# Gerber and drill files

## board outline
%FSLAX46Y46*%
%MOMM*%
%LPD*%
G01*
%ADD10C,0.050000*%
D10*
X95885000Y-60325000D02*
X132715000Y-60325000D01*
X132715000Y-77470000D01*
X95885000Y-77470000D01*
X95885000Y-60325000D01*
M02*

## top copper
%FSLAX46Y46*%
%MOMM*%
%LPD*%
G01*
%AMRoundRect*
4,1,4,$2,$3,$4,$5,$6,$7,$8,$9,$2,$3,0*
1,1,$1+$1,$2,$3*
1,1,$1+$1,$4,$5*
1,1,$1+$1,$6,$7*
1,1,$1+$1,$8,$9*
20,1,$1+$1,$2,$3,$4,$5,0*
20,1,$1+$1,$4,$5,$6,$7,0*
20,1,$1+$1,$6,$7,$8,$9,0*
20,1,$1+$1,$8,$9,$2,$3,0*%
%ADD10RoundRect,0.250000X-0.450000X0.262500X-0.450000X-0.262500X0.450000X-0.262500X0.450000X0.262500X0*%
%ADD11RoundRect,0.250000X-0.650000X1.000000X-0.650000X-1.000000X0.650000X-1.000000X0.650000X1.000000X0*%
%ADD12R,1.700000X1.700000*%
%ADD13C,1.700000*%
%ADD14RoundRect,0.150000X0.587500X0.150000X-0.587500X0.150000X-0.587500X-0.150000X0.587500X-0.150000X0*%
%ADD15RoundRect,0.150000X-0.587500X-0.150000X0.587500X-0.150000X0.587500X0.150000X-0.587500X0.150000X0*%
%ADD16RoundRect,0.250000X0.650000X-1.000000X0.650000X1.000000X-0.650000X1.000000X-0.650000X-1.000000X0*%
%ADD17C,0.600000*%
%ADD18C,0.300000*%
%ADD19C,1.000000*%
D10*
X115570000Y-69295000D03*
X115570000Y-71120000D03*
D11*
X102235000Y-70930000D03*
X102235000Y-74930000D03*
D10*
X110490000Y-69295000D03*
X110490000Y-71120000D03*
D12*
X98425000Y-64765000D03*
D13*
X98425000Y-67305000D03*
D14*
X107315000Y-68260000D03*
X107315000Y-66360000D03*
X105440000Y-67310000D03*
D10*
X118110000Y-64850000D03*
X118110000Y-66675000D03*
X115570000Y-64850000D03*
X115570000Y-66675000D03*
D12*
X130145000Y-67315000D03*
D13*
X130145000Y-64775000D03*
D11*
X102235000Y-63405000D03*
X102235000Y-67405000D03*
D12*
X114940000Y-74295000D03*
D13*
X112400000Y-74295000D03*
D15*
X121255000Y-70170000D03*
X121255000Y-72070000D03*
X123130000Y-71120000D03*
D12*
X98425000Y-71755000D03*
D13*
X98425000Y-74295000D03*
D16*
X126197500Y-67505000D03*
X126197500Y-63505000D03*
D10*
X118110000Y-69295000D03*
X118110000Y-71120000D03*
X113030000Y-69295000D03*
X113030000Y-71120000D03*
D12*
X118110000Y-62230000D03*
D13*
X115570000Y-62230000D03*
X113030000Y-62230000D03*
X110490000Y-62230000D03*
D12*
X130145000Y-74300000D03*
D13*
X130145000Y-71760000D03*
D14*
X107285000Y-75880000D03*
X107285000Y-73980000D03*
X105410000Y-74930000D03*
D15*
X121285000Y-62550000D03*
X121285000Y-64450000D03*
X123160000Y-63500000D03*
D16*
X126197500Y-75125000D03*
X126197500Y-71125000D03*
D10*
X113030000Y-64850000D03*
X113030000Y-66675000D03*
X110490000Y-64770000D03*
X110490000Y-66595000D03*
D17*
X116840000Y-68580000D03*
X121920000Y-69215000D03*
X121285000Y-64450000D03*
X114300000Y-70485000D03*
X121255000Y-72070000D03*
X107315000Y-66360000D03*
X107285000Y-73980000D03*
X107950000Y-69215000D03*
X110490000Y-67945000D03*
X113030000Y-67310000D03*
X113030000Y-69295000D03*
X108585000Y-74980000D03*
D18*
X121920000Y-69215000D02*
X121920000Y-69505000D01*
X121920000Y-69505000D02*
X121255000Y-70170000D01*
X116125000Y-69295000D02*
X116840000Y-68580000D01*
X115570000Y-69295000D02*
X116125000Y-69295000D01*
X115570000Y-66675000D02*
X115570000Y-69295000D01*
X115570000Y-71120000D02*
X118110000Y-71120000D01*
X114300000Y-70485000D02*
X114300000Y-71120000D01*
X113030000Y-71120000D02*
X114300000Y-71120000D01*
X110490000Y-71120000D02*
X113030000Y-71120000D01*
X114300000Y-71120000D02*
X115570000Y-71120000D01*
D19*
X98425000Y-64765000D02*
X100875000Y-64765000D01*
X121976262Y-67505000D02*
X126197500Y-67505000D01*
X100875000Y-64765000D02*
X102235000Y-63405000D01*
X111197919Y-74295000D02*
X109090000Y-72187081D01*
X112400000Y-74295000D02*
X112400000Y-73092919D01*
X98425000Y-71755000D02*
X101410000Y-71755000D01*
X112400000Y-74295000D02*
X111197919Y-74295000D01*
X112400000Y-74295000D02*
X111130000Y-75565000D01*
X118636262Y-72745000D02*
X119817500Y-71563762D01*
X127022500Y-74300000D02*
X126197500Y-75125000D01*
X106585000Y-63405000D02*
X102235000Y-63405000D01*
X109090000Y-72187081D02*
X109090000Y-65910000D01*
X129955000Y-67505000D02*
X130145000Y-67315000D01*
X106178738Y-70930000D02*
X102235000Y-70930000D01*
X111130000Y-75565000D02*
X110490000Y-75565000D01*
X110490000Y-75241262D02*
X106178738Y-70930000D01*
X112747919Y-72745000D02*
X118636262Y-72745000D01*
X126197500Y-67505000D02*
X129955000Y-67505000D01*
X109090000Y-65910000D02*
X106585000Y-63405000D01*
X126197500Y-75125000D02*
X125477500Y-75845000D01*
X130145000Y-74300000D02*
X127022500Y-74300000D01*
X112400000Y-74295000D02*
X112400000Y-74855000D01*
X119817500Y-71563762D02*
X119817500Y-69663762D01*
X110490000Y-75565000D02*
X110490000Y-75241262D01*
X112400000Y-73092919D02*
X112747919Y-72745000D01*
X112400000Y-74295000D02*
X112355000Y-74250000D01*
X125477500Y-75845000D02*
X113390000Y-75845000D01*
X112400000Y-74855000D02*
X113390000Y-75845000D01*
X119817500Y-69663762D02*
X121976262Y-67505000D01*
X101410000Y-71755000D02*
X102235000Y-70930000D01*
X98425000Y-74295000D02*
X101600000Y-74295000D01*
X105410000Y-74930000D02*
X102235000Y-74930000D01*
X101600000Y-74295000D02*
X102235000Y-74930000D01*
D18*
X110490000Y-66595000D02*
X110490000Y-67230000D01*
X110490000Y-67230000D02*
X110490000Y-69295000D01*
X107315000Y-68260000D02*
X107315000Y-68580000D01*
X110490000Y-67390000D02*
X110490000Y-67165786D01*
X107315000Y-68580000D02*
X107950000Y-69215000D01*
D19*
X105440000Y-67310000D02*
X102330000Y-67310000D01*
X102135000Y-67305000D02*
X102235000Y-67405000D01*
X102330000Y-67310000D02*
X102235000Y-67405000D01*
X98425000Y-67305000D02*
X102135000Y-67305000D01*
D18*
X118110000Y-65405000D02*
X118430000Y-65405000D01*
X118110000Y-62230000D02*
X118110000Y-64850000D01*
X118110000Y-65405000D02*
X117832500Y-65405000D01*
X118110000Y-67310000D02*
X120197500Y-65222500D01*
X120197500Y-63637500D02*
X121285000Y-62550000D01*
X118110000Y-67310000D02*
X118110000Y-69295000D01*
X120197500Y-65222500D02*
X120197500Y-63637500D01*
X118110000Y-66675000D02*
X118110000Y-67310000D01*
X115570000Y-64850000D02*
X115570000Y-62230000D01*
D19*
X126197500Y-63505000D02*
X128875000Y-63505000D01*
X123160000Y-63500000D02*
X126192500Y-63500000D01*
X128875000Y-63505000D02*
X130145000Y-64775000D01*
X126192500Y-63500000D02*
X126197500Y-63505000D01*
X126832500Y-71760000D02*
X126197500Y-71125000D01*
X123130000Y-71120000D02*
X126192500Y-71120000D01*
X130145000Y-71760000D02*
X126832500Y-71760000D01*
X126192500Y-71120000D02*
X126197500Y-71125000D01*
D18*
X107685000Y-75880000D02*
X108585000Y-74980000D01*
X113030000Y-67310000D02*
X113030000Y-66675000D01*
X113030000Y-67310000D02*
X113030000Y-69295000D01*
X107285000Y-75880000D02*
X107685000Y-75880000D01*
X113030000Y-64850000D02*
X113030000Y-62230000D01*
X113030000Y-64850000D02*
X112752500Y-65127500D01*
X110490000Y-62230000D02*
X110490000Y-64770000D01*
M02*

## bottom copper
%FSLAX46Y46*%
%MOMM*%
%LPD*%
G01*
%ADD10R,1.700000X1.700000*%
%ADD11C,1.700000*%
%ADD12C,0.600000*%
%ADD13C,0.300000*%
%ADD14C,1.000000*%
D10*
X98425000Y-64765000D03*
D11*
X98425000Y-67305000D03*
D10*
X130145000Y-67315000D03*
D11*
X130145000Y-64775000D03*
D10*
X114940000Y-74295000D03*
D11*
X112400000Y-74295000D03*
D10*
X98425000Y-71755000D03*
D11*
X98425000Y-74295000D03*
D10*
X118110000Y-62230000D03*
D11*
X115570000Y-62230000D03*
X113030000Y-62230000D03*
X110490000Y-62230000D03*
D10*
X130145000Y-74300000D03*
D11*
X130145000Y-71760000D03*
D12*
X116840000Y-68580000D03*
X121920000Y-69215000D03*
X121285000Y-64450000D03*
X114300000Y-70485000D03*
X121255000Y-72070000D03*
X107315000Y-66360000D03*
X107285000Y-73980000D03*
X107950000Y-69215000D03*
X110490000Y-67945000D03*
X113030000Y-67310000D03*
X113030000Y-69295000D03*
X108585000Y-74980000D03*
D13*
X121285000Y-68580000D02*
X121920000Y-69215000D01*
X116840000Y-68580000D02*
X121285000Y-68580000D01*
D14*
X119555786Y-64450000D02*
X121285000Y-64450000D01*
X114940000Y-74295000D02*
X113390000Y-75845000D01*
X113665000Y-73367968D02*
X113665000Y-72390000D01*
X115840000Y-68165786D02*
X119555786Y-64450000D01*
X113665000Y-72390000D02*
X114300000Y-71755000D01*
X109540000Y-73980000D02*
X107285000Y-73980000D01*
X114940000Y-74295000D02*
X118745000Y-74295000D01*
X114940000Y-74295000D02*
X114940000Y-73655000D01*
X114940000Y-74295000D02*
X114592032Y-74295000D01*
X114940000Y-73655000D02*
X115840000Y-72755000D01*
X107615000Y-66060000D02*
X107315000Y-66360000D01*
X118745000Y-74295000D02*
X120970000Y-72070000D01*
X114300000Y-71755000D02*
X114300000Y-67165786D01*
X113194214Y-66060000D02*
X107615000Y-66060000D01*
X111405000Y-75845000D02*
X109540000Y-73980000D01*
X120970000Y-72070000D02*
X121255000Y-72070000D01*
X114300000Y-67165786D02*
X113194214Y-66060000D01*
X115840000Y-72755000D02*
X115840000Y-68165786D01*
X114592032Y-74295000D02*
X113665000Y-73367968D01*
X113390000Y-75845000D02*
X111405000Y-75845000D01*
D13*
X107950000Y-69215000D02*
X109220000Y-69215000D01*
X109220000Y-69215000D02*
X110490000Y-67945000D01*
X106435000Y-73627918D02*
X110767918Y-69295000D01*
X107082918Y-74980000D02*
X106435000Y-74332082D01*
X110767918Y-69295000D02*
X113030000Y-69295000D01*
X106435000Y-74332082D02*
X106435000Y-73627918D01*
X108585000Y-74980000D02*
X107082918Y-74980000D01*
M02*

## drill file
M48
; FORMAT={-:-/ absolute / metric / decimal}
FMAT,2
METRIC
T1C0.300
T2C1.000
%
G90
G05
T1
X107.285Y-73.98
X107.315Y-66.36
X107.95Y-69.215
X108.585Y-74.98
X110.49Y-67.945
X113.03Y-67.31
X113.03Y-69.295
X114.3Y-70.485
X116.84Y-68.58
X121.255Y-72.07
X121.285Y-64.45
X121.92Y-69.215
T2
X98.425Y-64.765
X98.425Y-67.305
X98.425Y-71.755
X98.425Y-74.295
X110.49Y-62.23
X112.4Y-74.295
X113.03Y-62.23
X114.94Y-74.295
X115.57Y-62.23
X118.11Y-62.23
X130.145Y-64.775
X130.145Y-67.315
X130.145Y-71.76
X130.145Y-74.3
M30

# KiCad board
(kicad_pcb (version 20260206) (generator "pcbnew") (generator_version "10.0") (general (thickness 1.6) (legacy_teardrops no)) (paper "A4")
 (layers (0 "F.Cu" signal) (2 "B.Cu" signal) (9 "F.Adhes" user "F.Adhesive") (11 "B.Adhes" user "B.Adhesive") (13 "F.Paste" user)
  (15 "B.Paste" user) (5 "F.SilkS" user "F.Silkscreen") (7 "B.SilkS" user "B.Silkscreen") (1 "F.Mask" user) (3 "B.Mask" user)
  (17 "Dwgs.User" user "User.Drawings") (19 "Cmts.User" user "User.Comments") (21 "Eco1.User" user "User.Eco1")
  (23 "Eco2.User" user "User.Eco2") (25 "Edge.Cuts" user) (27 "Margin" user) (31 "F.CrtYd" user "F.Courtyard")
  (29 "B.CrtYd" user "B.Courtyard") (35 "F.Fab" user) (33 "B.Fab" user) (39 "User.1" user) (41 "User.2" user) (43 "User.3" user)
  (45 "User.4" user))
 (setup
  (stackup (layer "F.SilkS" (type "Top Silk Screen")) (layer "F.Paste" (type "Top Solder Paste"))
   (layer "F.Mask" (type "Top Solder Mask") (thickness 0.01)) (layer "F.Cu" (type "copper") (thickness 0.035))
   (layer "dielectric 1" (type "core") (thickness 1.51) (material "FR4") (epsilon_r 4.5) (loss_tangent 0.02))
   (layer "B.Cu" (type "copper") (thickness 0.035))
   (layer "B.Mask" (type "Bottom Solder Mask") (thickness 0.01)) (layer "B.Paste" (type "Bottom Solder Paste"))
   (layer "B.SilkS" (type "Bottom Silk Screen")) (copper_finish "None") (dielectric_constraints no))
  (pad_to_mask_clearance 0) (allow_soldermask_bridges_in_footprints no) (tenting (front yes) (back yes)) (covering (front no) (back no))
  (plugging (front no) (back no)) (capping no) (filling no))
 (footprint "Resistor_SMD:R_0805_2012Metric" (layer "F.Cu") (at 115.57 70.2075 -90)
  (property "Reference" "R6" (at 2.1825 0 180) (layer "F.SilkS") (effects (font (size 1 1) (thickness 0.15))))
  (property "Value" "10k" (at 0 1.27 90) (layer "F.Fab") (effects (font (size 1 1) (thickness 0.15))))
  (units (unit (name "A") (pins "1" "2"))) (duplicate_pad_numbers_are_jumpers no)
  (pad "1" smd roundrect (at -0.9125 0 270) (size 1.025 1.4) (layers "F.Cu" "F.Mask" "F.Paste") (roundrect_rratio 0.243902)
   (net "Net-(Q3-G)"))
  (pad "2" smd roundrect (at 0.9125 0 270) (size 1.025 1.4) (layers "F.Cu" "F.Mask" "F.Paste") (roundrect_rratio 0.243902) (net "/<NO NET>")))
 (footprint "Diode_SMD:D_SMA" (layer "F.Cu") (at 102.235 72.93 -90)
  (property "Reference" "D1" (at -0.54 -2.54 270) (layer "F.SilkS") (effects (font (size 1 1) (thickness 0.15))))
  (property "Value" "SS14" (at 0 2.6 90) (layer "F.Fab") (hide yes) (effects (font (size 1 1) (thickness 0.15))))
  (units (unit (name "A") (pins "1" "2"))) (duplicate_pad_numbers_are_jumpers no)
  (pad "1" smd roundrect (at -2 0 270) (size 2.5 1.8) (layers "F.Cu" "F.Mask" "F.Paste") (roundrect_rratio 0.1388888889) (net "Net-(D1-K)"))
  (pad "2" smd roundrect (at 2 0 270) (size 2.5 1.8) (layers "F.Cu" "F.Mask" "F.Paste") (roundrect_rratio 0.1388888889) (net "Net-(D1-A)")))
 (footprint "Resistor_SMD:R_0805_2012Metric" (layer "F.Cu") (at 110.49 70.2075 -90)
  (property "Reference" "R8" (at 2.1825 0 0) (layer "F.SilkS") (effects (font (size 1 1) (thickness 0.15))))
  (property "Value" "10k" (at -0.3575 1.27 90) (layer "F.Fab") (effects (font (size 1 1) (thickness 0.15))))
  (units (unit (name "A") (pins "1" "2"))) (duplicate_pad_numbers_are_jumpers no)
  (pad "1" smd roundrect (at -0.9125 0 270) (size 1.025 1.4) (layers "F.Cu" "F.Mask" "F.Paste") (roundrect_rratio 0.243902)
   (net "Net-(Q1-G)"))
  (pad "2" smd roundrect (at 0.9125 0 270) (size 1.025 1.4) (layers "F.Cu" "F.Mask" "F.Paste") (roundrect_rratio 0.243902) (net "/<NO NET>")))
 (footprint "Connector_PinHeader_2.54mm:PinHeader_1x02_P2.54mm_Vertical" (layer "F.Cu") (at 98.425 64.765)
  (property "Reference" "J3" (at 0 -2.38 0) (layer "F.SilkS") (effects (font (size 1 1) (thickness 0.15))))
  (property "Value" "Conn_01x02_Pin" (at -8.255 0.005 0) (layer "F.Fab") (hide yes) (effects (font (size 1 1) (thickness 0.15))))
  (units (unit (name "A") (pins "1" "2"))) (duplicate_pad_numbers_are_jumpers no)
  (pad "1" thru_hole rect (at 0 0) (size 1.7 1.7) (drill 1) (layers "*.Cu" "*.Mask") (remove_unused_layers no) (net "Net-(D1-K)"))
  (pad "2" thru_hole circle (at 0 2.54) (size 1.7 1.7) (drill 1) (layers "*.Cu" "*.Mask") (remove_unused_layers no) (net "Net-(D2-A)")))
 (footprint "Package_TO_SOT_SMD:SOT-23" (layer "F.Cu") (at 106.3775 67.31 180)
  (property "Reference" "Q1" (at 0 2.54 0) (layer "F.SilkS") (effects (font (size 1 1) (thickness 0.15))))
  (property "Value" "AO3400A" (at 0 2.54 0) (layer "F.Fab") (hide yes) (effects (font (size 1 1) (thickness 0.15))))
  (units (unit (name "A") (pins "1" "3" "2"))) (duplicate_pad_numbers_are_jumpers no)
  (pad "1" smd roundrect (at -0.9375 -0.95 180) (size 1.475 0.6) (layers "F.Cu" "F.Mask" "F.Paste") (roundrect_rratio 0.25)
   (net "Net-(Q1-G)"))
  (pad "2" smd roundrect (at -0.9375 0.95 180) (size 1.475 0.6) (layers "F.Cu" "F.Mask" "F.Paste") (roundrect_rratio 0.25) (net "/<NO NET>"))
  (pad "3" smd roundrect (at 0.9375 0 180) (size 1.475 0.6) (layers "F.Cu" "F.Mask" "F.Paste") (roundrect_rratio 0.25) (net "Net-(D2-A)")))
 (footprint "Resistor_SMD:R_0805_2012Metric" (layer "F.Cu") (at 118.11 65.7625 -90)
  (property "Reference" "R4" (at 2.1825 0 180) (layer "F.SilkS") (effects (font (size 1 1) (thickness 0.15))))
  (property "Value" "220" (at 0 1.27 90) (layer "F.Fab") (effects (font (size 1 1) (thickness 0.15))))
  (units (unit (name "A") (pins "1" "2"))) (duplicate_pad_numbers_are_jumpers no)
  (pad "1" smd roundrect (at -0.9125 0 270) (size 1.025 1.4) (layers "F.Cu" "F.Mask" "F.Paste") (roundrect_rratio 0.243902)
   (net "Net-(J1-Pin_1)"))
  (pad "2" smd roundrect (at 0.9125 0 270) (size 1.025 1.4) (layers "F.Cu" "F.Mask" "F.Paste") (roundrect_rratio 0.243902)
   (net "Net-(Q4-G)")))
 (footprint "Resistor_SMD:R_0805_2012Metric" (layer "F.Cu") (at 115.57 65.7625 -90)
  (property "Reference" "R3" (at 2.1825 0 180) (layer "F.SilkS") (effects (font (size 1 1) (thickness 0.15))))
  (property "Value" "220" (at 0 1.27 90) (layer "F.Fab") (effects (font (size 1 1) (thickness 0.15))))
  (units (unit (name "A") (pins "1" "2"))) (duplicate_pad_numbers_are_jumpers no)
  (pad "1" smd roundrect (at -0.9125 0 270) (size 1.025 1.4) (layers "F.Cu" "F.Mask" "F.Paste") (roundrect_rratio 0.243902)
   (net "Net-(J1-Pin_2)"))
  (pad "2" smd roundrect (at 0.9125 0 270) (size 1.025 1.4) (layers "F.Cu" "F.Mask" "F.Paste") (roundrect_rratio 0.243902)
   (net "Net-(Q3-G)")))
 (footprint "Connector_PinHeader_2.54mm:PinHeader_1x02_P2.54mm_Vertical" (layer "F.Cu") (at 130.145 67.315 180)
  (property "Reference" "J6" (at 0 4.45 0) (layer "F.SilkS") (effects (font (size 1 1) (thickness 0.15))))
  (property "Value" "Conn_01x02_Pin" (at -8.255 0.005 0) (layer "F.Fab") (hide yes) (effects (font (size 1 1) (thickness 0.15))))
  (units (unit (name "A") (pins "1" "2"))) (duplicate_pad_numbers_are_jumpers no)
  (pad "1" thru_hole rect (at 0 0 180) (size 1.7 1.7) (drill 1) (layers "*.Cu" "*.Mask") (remove_unused_layers no) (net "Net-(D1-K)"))
  (pad "2" thru_hole circle (at 0 2.54 180) (size 1.7 1.7) (drill 1) (layers "*.Cu" "*.Mask") (remove_unused_layers no) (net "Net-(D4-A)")))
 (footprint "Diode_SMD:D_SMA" (layer "F.Cu") (at 102.235 65.405 -90)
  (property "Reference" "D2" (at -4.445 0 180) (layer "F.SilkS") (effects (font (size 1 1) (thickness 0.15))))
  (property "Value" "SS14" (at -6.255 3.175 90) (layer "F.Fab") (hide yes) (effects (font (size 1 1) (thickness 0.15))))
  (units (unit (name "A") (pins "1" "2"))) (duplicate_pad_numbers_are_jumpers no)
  (pad "1" smd roundrect (at -2 0 270) (size 2.5 1.8) (layers "F.Cu" "F.Mask" "F.Paste") (roundrect_rratio 0.1388888889) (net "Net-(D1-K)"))
  (pad "2" smd roundrect (at 2 0 270) (size 2.5 1.8) (layers "F.Cu" "F.Mask" "F.Paste") (roundrect_rratio 0.1388888889) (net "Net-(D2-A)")))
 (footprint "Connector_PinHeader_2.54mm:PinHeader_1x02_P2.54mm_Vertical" (layer "F.Cu") (at 114.94 74.295 -90)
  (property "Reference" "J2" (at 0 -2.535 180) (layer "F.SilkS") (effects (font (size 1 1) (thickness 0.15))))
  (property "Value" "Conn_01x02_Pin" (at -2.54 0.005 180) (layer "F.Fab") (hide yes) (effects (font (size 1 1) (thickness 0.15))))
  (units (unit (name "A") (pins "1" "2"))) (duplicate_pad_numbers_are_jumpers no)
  (pad "1" thru_hole rect (at 0 0 270) (size 1.7 1.7) (drill 1) (layers "*.Cu" "*.Mask") (remove_unused_layers no) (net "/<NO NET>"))
  (pad "2" thru_hole circle (at 0 2.54 270) (size 1.7 1.7) (drill 1) (layers "*.Cu" "*.Mask") (remove_unused_layers no) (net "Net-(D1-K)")))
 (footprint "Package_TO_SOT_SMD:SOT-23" (layer "F.Cu") (at 122.1925 71.12)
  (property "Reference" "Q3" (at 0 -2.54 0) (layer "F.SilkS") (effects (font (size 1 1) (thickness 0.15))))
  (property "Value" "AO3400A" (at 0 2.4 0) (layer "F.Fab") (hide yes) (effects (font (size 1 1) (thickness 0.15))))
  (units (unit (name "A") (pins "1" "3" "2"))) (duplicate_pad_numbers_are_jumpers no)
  (pad "1" smd roundrect (at -0.9375 -0.95) (size 1.475 0.6) (layers "F.Cu" "F.Mask" "F.Paste") (roundrect_rratio 0.25) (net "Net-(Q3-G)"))
  (pad "2" smd roundrect (at -0.9375 0.95) (size 1.475 0.6) (layers "F.Cu" "F.Mask" "F.Paste") (roundrect_rratio 0.25) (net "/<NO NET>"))
  (pad "3" smd roundrect (at 0.9375 0) (size 1.475 0.6) (layers "F.Cu" "F.Mask" "F.Paste") (roundrect_rratio 0.25) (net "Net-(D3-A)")))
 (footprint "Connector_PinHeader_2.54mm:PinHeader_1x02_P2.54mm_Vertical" (layer "F.Cu") (at 98.425 71.755)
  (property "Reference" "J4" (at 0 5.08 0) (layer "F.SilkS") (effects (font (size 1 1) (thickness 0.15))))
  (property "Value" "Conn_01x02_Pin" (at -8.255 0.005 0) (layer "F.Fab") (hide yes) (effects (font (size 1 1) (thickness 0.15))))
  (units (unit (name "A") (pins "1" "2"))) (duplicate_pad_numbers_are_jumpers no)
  (pad "1" thru_hole rect (at 0 0) (size 1.7 1.7) (drill 1) (layers "*.Cu" "*.Mask") (remove_unused_layers no) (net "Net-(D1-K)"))
  (pad "2" thru_hole circle (at 0 2.54) (size 1.7 1.7) (drill 1) (layers "*.Cu" "*.Mask") (remove_unused_layers no) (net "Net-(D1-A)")))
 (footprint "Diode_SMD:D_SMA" (layer "F.Cu") (at 126.1975 65.505 90)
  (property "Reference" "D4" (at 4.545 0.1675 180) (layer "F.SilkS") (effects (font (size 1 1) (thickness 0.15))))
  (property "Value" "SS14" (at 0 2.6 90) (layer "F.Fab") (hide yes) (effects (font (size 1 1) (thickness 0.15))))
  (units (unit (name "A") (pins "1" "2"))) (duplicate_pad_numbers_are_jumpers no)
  (pad "1" smd roundrect (at -2 0 90) (size 2.5 1.8) (layers "F.Cu" "F.Mask" "F.Paste") (roundrect_rratio 0.1388888889) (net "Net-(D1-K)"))
  (pad "2" smd roundrect (at 2 0 90) (size 2.5 1.8) (layers "F.Cu" "F.Mask" "F.Paste") (roundrect_rratio 0.1388888889) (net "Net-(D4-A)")))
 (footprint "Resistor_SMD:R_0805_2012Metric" (layer "F.Cu") (at 118.11 70.2075 -90)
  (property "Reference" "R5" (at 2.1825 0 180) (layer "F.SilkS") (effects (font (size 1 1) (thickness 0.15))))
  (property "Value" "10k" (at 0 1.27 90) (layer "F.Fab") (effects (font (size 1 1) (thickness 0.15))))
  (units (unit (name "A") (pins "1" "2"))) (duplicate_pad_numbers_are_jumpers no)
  (pad "1" smd roundrect (at -0.9125 0 270) (size 1.025 1.4) (layers "F.Cu" "F.Mask" "F.Paste") (roundrect_rratio 0.243902)
   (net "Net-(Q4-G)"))
  (pad "2" smd roundrect (at 0.9125 0 270) (size 1.025 1.4) (layers "F.Cu" "F.Mask" "F.Paste") (roundrect_rratio 0.243902) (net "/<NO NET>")))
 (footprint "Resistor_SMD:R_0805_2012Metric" (layer "F.Cu") (at 113.03 70.2075 -90)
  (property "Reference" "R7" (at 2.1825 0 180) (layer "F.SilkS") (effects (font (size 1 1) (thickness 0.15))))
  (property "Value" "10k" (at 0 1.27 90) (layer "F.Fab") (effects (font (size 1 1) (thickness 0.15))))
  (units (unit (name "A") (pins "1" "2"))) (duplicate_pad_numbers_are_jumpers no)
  (pad "1" smd roundrect (at -0.9125 0 270) (size 1.025 1.4) (layers "F.Cu" "F.Mask" "F.Paste") (roundrect_rratio 0.243902)
   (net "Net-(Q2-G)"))
  (pad "2" smd roundrect (at 0.9125 0 270) (size 1.025 1.4) (layers "F.Cu" "F.Mask" "F.Paste") (roundrect_rratio 0.243902) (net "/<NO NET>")))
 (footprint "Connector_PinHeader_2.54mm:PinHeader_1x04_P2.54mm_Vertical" (layer "F.Cu") (at 118.11 62.23 -90)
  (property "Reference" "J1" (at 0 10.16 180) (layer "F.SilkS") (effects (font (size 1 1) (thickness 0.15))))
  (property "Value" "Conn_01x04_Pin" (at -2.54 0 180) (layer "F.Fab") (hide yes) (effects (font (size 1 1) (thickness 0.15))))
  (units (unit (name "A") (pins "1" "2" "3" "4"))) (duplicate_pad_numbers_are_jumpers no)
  (pad "1" thru_hole rect (at 0 0 270) (size 1.7 1.7) (drill 1) (layers "*.Cu" "*.Mask") (remove_unused_layers no) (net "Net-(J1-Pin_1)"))
  (pad "2" thru_hole circle (at 0 2.54 270) (size 1.7 1.7) (drill 1) (layers "*.Cu" "*.Mask") (remove_unused_layers no)
   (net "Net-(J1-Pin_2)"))
  (pad "3" thru_hole circle (at 0 5.08 270) (size 1.7 1.7) (drill 1) (layers "*.Cu" "*.Mask") (remove_unused_layers no)
   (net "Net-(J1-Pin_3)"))
  (pad "4" thru_hole circle (at 0 7.62 270) (size 1.7 1.7) (drill 1) (layers "*.Cu" "*.Mask") (remove_unused_layers no)
   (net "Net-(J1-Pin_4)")))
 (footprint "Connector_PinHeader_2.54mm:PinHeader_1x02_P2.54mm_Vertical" (layer "F.Cu") (at 130.145 74.3 180)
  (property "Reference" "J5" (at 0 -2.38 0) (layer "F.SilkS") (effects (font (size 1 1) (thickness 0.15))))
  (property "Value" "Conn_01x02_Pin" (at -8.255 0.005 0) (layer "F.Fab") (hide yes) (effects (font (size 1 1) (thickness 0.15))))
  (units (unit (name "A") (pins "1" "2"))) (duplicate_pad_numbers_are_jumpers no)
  (pad "1" thru_hole rect (at 0 0 180) (size 1.7 1.7) (drill 1) (layers "*.Cu" "*.Mask") (remove_unused_layers no) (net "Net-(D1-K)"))
  (pad "2" thru_hole circle (at 0 2.54 180) (size 1.7 1.7) (drill 1) (layers "*.Cu" "*.Mask") (remove_unused_layers no) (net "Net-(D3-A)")))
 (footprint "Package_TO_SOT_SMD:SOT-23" (layer "F.Cu") (at 106.3475 74.93 180)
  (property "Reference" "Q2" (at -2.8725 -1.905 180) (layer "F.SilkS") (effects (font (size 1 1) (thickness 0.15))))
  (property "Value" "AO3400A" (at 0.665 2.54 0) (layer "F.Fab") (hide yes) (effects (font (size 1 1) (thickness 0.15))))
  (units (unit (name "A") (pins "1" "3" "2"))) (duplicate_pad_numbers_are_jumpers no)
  (pad "1" smd roundrect (at -0.9375 -0.95 180) (size 1.475 0.6) (layers "F.Cu" "F.Mask" "F.Paste") (roundrect_rratio 0.25)
   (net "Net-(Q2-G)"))
  (pad "2" smd roundrect (at -0.9375 0.95 180) (size 1.475 0.6) (layers "F.Cu" "F.Mask" "F.Paste") (roundrect_rratio 0.25) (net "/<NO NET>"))
  (pad "3" smd roundrect (at 0.9375 0 180) (size 1.475 0.6) (layers "F.Cu" "F.Mask" "F.Paste") (roundrect_rratio 0.25) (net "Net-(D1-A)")))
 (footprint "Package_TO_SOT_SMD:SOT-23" (layer "F.Cu") (at 122.2225 63.5)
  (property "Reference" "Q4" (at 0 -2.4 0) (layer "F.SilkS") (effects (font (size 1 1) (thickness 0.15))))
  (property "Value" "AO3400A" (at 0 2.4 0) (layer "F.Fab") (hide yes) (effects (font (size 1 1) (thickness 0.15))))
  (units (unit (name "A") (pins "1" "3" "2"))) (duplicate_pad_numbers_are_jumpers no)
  (pad "1" smd roundrect (at -0.9375 -0.95) (size 1.475 0.6) (layers "F.Cu" "F.Mask" "F.Paste") (roundrect_rratio 0.25) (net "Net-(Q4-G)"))
  (pad "2" smd roundrect (at -0.9375 0.95) (size 1.475 0.6) (layers "F.Cu" "F.Mask" "F.Paste") (roundrect_rratio 0.25) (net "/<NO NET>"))
  (pad "3" smd roundrect (at 0.9375 0) (size 1.475 0.6) (layers "F.Cu" "F.Mask" "F.Paste") (roundrect_rratio 0.25) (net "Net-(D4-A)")))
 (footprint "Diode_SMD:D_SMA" (layer "F.Cu") (at 126.1975 73.125 90)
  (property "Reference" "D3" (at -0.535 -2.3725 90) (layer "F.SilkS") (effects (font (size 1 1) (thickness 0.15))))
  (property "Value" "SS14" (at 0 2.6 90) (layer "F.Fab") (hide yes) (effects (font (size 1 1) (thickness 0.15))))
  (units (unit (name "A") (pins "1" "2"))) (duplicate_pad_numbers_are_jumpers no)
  (pad "1" smd roundrect (at -2 0 90) (size 2.5 1.8) (layers "F.Cu" "F.Mask" "F.Paste") (roundrect_rratio 0.1388888889) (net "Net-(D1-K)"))
  (pad "2" smd roundrect (at 2 0 90) (size 2.5 1.8) (layers "F.Cu" "F.Mask" "F.Paste") (roundrect_rratio 0.1388888889) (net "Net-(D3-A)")))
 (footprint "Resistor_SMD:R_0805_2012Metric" (layer "F.Cu") (at 113.03 65.7625 -90)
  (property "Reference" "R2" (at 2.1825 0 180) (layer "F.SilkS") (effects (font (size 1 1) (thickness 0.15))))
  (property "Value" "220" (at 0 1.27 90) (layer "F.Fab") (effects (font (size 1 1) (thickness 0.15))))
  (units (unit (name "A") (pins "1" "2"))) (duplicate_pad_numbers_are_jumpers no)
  (pad "1" smd roundrect (at -0.9125 0 270) (size 1.025 1.4) (layers "F.Cu" "F.Mask" "F.Paste") (roundrect_rratio 0.243902)
   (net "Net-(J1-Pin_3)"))
  (pad "2" smd roundrect (at 0.9125 0 270) (size 1.025 1.4) (layers "F.Cu" "F.Mask" "F.Paste") (roundrect_rratio 0.243902)
   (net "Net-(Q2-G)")))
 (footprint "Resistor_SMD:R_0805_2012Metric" (layer "F.Cu") (at 110.49 65.6825 -90)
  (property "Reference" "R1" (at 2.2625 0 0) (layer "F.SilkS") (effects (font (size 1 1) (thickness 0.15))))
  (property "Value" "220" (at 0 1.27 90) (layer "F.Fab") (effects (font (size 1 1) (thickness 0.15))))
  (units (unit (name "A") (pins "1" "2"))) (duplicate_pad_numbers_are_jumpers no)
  (pad "1" smd roundrect (at -0.9125 0 270) (size 1.025 1.4) (layers "F.Cu" "F.Mask" "F.Paste") (roundrect_rratio 0.243902)
   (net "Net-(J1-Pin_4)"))
  (pad "2" smd roundrect (at 0.9125 0 270) (size 1.025 1.4) (layers "F.Cu" "F.Mask" "F.Paste") (roundrect_rratio 0.243902)
   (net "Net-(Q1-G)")))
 (gr_rect (start 95.885 60.325) (end 132.715 77.47) (stroke (width 0.05) (type default)) (fill no) (layer "Edge.Cuts"))
 (segment (start 121.92 69.215) (end 121.92 69.505) (width 0.3) (layer "F.Cu") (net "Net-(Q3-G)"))
 (segment (start 121.92 69.505) (end 121.255 70.17) (width 0.3) (layer "F.Cu") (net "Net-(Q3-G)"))
 (segment (start 116.125 69.295) (end 116.84 68.58) (width 0.3) (layer "F.Cu") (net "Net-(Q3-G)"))
 (segment (start 115.57 69.295) (end 116.125 69.295) (width 0.3) (layer "F.Cu") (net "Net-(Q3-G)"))
 (segment (start 115.57 66.675) (end 115.57 69.295) (width 0.3) (layer "F.Cu") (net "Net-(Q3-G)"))
 (via (at 116.84 68.58) (size 0.6) (drill 0.3) (layers "F.Cu" "B.Cu") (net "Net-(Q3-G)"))
 (via (at 121.92 69.215) (size 0.6) (drill 0.3) (layers "F.Cu" "B.Cu") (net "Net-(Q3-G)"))
 (segment (start 121.285 68.58) (end 121.92 69.215) (width 0.3) (layer "B.Cu") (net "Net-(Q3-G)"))
 (segment (start 116.84 68.58) (end 121.285 68.58) (width 0.3) (layer "B.Cu") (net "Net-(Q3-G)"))
 (segment (start 115.57 71.12) (end 118.11 71.12) (width 0.3) (layer "F.Cu") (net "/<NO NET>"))
 (segment (start 114.3 70.485) (end 114.3 71.12) (width 0.3) (layer "F.Cu") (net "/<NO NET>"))
 (segment (start 113.03 71.12) (end 114.3 71.12) (width 0.3) (layer "F.Cu") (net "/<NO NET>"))
 (segment (start 110.49 71.12) (end 113.03 71.12) (width 0.3) (layer "F.Cu") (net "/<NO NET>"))
 (segment (start 114.3 71.12) (end 115.57 71.12) (width 0.3) (layer "F.Cu") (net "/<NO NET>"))
 (via (at 121.285 64.45) (size 0.6) (drill 0.3) (layers "F.Cu" "B.Cu") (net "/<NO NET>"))
 (via (at 114.3 70.485) (size 0.6) (drill 0.3) (layers "F.Cu" "B.Cu") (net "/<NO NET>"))
 (via (at 121.255 72.07) (size 0.6) (drill 0.3) (layers "F.Cu" "B.Cu") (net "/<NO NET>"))
 (via (at 107.315 66.36) (size 0.6) (drill 0.3) (layers "F.Cu" "B.Cu") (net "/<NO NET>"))
 (via (at 107.285 73.98) (size 0.6) (drill 0.3) (layers "F.Cu" "B.Cu") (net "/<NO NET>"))
 (segment (start 119.555786 64.45) (end 121.285 64.45) (width 1) (layer "B.Cu") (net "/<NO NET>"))
 (segment (start 114.94 74.295) (end 113.39 75.845) (width 1) (layer "B.Cu") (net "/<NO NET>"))
 (segment (start 113.665 73.367968) (end 113.665 72.39) (width 1) (layer "B.Cu") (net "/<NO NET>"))
 (segment (start 115.84 68.165786) (end 119.555786 64.45) (width 1) (layer "B.Cu") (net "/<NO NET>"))
 (segment (start 113.665 72.39) (end 114.3 71.755) (width 1) (layer "B.Cu") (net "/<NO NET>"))
 (segment (start 109.54 73.98) (end 107.285 73.98) (width 1) (layer "B.Cu") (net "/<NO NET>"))
 (segment (start 114.94 74.295) (end 118.745 74.295) (width 1) (layer "B.Cu") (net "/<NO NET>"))
 (segment (start 114.94 74.295) (end 114.94 73.655) (width 1) (layer "B.Cu") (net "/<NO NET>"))
 (segment (start 114.94 74.295) (end 114.592032 74.295) (width 1) (layer "B.Cu") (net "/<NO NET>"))
 (segment (start 114.94 73.655) (end 115.84 72.755) (width 1) (layer "B.Cu") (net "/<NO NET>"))
 (segment (start 107.615 66.06) (end 107.315 66.36) (width 1) (layer "B.Cu") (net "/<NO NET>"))
 (segment (start 118.745 74.295) (end 120.97 72.07) (width 1) (layer "B.Cu") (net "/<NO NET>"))
 (segment (start 114.3 71.755) (end 114.3 67.165786) (width 1) (layer "B.Cu") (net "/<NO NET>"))
 (segment (start 113.194214 66.06) (end 107.615 66.06) (width 1) (layer "B.Cu") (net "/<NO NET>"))
 (segment (start 111.405 75.845) (end 109.54 73.98) (width 1) (layer "B.Cu") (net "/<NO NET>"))
 (segment (start 120.97 72.07) (end 121.255 72.07) (width 1) (layer "B.Cu") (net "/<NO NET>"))
 (segment (start 114.3 67.165786) (end 113.194214 66.06) (width 1) (layer "B.Cu") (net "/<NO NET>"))
 (segment (start 115.84 72.755) (end 115.84 68.165786) (width 1) (layer "B.Cu") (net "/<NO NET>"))
 (segment (start 114.592032 74.295) (end 113.665 73.367968) (width 1) (layer "B.Cu") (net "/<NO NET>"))
 (segment (start 113.39 75.845) (end 111.405 75.845) (width 1) (layer "B.Cu") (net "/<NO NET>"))
 (segment (start 98.425 64.765) (end 100.875 64.765) (width 1) (layer "F.Cu") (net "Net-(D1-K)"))
 (segment (start 121.976262 67.505) (end 126.1975 67.505) (width 1) (layer "F.Cu") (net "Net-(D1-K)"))
 (segment (start 100.875 64.765) (end 102.235 63.405) (width 1) (layer "F.Cu") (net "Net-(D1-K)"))
 (segment (start 111.197919 74.295) (end 109.09 72.187081) (width 1) (layer "F.Cu") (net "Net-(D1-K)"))
 (segment (start 112.4 74.295) (end 112.4 73.092919) (width 1) (layer "F.Cu") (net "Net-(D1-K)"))
 (segment (start 98.425 71.755) (end 101.41 71.755) (width 1) (layer "F.Cu") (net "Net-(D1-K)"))
 (segment (start 112.4 74.295) (end 111.197919 74.295) (width 1) (layer "F.Cu") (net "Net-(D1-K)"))
 (segment (start 112.4 74.295) (end 111.13 75.565) (width 1) (layer "F.Cu") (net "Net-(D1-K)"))
 (segment (start 118.636262 72.745) (end 119.8175 71.563762) (width 1) (layer "F.Cu") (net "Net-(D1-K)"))
 (segment (start 127.0225 74.3) (end 126.1975 75.125) (width 1) (layer "F.Cu") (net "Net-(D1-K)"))
 (segment (start 106.585 63.405) (end 102.235 63.405) (width 1) (layer "F.Cu") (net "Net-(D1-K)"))
 (segment (start 109.09 72.187081) (end 109.09 65.91) (width 1) (layer "F.Cu") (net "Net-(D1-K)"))
 (segment (start 129.955 67.505) (end 130.145 67.315) (width 1) (layer "F.Cu") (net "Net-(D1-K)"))
 (segment (start 106.178738 70.93) (end 102.235 70.93) (width 1) (layer "F.Cu") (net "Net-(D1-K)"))
 (segment (start 111.13 75.565) (end 110.49 75.565) (width 1) (layer "F.Cu") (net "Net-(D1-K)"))
 (segment (start 110.49 75.241262) (end 106.178738 70.93) (width 1) (layer "F.Cu") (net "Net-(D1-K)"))
 (segment (start 112.747919 72.745) (end 118.636262 72.745) (width 1) (layer "F.Cu") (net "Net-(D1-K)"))
 (segment (start 126.1975 67.505) (end 129.955 67.505) (width 1) (layer "F.Cu") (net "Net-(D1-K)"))
 (segment (start 109.09 65.91) (end 106.585 63.405) (width 1) (layer "F.Cu") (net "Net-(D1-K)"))
 (segment (start 126.1975 75.125) (end 125.4775 75.845) (width 1) (layer "F.Cu") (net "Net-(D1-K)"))
 (segment (start 130.145 74.3) (end 127.0225 74.3) (width 1) (layer "F.Cu") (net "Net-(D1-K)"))
 (segment (start 112.4 74.295) (end 112.4 74.855) (width 1) (layer "F.Cu") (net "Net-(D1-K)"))
 (segment (start 119.8175 71.563762) (end 119.8175 69.663762) (width 1) (layer "F.Cu") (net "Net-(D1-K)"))
 (segment (start 110.49 75.565) (end 110.49 75.241262) (width 1) (layer "F.Cu") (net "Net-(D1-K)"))
 (segment (start 112.4 73.092919) (end 112.747919 72.745) (width 1) (layer "F.Cu") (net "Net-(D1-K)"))
 (segment (start 112.4 74.295) (end 112.355 74.25) (width 1) (layer "F.Cu") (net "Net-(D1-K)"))
 (segment (start 125.4775 75.845) (end 113.39 75.845) (width 1) (layer "F.Cu") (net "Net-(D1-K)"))
 (segment (start 112.4 74.855) (end 113.39 75.845) (width 1) (layer "F.Cu") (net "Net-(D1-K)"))
 (segment (start 119.8175 69.663762) (end 121.976262 67.505) (width 1) (layer "F.Cu") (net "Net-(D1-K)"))
 (segment (start 101.41 71.755) (end 102.235 70.93) (width 1) (layer "F.Cu") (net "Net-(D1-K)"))
 (segment (start 98.425 74.295) (end 101.6 74.295) (width 1) (layer "F.Cu") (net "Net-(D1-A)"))
 (segment (start 105.41 74.93) (end 102.235 74.93) (width 1) (layer "F.Cu") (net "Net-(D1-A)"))
 (segment (start 101.6 74.295) (end 102.235 74.93) (width 1) (layer "F.Cu") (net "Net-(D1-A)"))
 (segment (start 110.49 66.595) (end 110.49 67.23) (width 0.3) (layer "F.Cu") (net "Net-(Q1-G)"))
 (segment (start 110.49 67.23) (end 110.49 69.295) (width 0.3) (layer "F.Cu") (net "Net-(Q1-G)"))
 (segment (start 107.315 68.26) (end 107.315 68.58) (width 0.3) (layer "F.Cu") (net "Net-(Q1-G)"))
 (segment (start 110.49 67.39) (end 110.49 67.165786) (width 0.3) (layer "F.Cu") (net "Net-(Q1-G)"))
 (segment (start 107.315 68.58) (end 107.95 69.215) (width 0.3) (layer "F.Cu") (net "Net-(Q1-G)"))
 (via (at 107.95 69.215) (size 0.6) (drill 0.3) (layers "F.Cu" "B.Cu") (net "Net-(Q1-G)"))
 (via (at 110.49 67.945) (size 0.6) (drill 0.3) (layers "F.Cu" "B.Cu") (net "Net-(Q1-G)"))
 (segment (start 107.95 69.215) (end 109.22 69.215) (width 0.3) (layer "B.Cu") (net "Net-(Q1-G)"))
 (segment (start 109.22 69.215) (end 110.49 67.945) (width 0.3) (layer "B.Cu") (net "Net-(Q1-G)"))
 (segment (start 105.44 67.31) (end 102.33 67.31) (width 1) (layer "F.Cu") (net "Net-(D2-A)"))
 (segment (start 102.135 67.305) (end 102.235 67.405) (width 1) (layer "F.Cu") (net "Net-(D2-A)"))
 (segment (start 102.33 67.31) (end 102.235 67.405) (width 1) (layer "F.Cu") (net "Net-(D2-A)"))
 (segment (start 98.425 67.305) (end 102.135 67.305) (width 1) (layer "F.Cu") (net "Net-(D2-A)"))
 (segment (start 118.11 65.405) (end 118.43 65.405) (width 0.3) (layer "F.Cu") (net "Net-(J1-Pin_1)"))
 (segment (start 118.11 62.23) (end 118.11 64.85) (width 0.3) (layer "F.Cu") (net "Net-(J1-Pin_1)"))
 (segment (start 118.11 65.405) (end 117.8325 65.405) (width 0.3) (layer "F.Cu") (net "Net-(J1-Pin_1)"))
 (segment (start 118.11 67.31) (end 120.1975 65.2225) (width 0.3) (layer "F.Cu") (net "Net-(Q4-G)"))
 (segment (start 120.1975 63.6375) (end 121.285 62.55) (width 0.3) (layer "F.Cu") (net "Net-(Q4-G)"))
 (segment (start 118.11 67.31) (end 118.11 69.295) (width 0.3) (layer "F.Cu") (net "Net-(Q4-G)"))
 (segment (start 120.1975 65.2225) (end 120.1975 63.6375) (width 0.3) (layer "F.Cu") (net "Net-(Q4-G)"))
 (segment (start 118.11 66.675) (end 118.11 67.31) (width 0.3) (layer "F.Cu") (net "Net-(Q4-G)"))
 (segment (start 115.57 64.85) (end 115.57 62.23) (width 0.3) (layer "F.Cu") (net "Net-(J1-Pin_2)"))
 (segment (start 126.1975 63.505) (end 128.875 63.505) (width 1) (layer "F.Cu") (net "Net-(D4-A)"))
 (segment (start 123.16 63.5) (end 126.1925 63.5) (width 1) (layer "F.Cu") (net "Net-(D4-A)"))
 (segment (start 128.875 63.505) (end 130.145 64.775) (width 1) (layer "F.Cu") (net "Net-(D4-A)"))
 (segment (start 126.1925 63.5) (end 126.1975 63.505) (width 1) (layer "F.Cu") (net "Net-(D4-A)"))
 (segment (start 126.8325 71.76) (end 126.1975 71.125) (width 1) (layer "F.Cu") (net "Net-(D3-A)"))
 (segment (start 123.13 71.12) (end 126.1925 71.12) (width 1) (layer "F.Cu") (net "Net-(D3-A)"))
 (segment (start 130.145 71.76) (end 126.8325 71.76) (width 1) (layer "F.Cu") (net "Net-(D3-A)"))
 (segment (start 126.1925 71.12) (end 126.1975 71.125) (width 1) (layer "F.Cu") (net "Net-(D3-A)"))
 (segment (start 107.685 75.88) (end 108.585 74.98) (width 0.3) (layer "F.Cu") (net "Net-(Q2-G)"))
 (segment (start 113.03 67.31) (end 113.03 66.675) (width 0.3) (layer "F.Cu") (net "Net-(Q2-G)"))
 (segment (start 113.03 67.31) (end 113.03 69.295) (width 0.3) (layer "F.Cu") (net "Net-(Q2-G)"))
 (segment (start 107.285 75.88) (end 107.685 75.88) (width 0.3) (layer "F.Cu") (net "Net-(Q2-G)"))
 (via (at 113.03 67.31) (size 0.6) (drill 0.3) (layers "F.Cu" "B.Cu") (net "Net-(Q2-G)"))
 (via (at 113.03 69.295) (size 0.6) (drill 0.3) (layers "F.Cu" "B.Cu") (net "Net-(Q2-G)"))
 (via (at 108.585 74.98) (size 0.6) (drill 0.3) (layers "F.Cu" "B.Cu") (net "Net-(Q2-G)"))
 (segment (start 106.435 73.627918) (end 110.767918 69.295) (width 0.3) (layer "B.Cu") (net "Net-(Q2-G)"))
 (segment (start 107.082918 74.98) (end 106.435 74.332082) (width 0.3) (layer "B.Cu") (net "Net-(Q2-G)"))
 (segment (start 110.767918 69.295) (end 113.03 69.295) (width 0.3) (layer "B.Cu") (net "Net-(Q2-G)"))
 (segment (start 106.435 74.332082) (end 106.435 73.627918) (width 0.3) (layer "B.Cu") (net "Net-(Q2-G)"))
 (segment (start 108.585 74.98) (end 107.082918 74.98) (width 0.3) (layer "B.Cu") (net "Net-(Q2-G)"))
 (segment (start 113.03 64.85) (end 113.03 62.23) (width 0.3) (layer "F.Cu") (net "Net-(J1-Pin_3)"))
 (segment (start 113.03 64.85) (end 112.7525 65.1275) (width 0.3) (layer "F.Cu") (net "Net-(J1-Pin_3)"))
 (segment (start 110.49 62.23) (end 110.49 64.77) (width 0.3) (layer "F.Cu") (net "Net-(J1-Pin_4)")))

